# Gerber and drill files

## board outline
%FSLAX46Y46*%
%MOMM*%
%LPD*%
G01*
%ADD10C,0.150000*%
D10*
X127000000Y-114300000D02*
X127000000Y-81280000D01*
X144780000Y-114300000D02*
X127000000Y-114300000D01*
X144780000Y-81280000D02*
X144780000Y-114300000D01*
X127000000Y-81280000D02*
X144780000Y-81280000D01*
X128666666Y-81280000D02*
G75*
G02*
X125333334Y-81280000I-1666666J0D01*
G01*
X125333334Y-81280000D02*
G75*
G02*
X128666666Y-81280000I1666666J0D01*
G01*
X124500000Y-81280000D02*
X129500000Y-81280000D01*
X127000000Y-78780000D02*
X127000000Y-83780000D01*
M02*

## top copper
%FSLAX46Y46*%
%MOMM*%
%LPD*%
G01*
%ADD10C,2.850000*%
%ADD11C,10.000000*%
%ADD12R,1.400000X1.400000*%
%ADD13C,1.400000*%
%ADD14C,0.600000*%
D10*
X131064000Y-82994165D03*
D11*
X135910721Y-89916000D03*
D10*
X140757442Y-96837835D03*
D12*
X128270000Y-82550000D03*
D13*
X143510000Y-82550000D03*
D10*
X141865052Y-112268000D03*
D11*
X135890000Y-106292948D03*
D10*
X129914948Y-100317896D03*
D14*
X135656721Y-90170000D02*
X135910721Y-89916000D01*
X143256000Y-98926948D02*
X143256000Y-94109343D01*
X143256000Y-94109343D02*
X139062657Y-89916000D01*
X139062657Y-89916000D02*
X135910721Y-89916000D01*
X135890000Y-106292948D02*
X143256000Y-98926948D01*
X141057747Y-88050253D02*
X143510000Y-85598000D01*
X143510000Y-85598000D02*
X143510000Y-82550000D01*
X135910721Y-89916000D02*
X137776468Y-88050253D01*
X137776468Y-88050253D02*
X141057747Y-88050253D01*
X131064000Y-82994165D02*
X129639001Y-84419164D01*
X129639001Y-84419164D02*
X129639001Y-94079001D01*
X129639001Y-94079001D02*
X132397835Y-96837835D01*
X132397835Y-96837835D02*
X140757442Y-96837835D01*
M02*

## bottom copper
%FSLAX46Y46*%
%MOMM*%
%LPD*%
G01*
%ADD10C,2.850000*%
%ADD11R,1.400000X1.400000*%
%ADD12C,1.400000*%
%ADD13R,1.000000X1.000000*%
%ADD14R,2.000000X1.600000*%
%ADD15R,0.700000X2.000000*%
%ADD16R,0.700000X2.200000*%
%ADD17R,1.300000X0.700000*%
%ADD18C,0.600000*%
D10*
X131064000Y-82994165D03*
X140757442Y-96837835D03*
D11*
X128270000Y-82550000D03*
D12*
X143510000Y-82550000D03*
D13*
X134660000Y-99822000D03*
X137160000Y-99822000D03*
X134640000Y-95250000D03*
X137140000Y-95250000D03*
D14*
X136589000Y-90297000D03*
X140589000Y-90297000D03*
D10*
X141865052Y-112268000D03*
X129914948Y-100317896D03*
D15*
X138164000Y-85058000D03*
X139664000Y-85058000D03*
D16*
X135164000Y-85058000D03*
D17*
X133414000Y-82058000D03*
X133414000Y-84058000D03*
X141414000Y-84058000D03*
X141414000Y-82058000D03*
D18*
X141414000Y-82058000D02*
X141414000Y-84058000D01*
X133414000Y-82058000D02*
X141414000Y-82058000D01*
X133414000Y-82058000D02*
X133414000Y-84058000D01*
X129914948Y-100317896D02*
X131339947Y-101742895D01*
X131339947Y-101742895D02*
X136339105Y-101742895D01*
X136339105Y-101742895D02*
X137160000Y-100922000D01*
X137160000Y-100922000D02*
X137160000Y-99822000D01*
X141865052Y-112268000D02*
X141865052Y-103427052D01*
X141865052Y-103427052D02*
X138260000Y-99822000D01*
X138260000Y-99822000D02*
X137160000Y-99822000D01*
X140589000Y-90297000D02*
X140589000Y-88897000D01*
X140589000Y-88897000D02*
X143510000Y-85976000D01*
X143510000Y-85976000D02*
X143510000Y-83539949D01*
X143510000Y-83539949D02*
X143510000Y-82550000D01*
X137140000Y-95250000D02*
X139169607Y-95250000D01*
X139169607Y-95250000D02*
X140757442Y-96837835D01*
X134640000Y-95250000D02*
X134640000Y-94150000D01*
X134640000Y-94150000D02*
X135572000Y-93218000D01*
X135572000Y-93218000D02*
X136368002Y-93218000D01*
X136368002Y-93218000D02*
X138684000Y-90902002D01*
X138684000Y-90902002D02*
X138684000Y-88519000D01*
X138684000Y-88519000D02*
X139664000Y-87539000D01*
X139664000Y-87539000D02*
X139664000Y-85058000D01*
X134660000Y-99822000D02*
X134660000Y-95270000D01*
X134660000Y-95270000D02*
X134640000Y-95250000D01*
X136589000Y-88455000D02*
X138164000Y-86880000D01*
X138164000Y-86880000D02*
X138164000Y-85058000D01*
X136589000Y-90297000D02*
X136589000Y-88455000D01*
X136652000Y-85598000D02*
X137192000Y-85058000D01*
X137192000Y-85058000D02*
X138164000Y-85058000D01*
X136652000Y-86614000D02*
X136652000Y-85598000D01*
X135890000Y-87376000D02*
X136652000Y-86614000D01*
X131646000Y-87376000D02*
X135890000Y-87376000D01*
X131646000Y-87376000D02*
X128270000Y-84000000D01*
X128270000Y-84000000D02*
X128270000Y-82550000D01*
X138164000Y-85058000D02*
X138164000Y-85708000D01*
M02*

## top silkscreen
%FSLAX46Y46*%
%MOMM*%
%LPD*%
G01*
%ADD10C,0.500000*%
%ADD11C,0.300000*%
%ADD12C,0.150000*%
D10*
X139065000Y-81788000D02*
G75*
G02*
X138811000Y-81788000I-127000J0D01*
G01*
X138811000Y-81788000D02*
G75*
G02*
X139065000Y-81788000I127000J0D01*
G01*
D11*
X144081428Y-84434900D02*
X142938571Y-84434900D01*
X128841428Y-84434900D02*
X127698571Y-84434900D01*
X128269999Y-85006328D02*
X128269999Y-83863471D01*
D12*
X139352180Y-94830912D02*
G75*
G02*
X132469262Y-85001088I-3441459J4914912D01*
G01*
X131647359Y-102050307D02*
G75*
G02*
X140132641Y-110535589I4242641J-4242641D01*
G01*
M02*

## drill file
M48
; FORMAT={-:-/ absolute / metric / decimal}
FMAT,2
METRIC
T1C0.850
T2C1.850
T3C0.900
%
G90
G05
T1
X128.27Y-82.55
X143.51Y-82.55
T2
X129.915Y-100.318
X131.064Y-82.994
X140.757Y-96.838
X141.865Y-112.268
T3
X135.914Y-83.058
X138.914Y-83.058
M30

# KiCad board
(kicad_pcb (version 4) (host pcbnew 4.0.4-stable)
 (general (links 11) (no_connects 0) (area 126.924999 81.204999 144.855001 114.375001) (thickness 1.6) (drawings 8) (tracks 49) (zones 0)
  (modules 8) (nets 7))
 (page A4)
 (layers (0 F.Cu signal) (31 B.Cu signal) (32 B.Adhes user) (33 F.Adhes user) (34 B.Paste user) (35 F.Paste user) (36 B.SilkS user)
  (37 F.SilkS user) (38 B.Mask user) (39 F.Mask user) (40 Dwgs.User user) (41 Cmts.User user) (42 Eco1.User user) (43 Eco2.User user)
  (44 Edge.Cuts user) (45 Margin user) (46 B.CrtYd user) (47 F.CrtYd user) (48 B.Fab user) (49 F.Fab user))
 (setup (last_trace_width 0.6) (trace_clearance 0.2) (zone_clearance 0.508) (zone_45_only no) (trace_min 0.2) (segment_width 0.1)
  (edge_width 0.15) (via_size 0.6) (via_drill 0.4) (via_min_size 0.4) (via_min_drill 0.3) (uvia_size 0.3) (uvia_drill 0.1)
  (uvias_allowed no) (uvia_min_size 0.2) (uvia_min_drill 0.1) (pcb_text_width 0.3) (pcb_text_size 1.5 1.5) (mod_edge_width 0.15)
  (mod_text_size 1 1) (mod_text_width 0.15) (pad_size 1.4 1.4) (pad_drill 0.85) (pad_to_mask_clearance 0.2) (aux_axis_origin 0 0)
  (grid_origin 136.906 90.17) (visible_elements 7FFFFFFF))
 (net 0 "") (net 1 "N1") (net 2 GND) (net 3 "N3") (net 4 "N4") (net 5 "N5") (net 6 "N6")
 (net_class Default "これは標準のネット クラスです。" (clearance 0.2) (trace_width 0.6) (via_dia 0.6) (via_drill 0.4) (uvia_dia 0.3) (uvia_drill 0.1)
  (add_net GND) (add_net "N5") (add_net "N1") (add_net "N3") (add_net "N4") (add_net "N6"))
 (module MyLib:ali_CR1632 (layer F.Cu) (at 135.910721 89.916 305)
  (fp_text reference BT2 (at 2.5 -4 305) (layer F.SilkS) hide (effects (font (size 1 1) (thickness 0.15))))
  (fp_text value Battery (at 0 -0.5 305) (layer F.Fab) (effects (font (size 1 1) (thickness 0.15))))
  (fp_arc (start 0 0) (end 6 0) (angle 180) (layer F.SilkS) (width 0.15))
  (pad 1 thru_hole circle (at -8.45 0 305) (size 2.85 2.85) (drill 1.85) (layers *.Cu *.Mask) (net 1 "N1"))
  (pad 2 smd circle (at 0 0 305) (size 10 10) (layers F.Cu F.Paste F.Mask) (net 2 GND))
  (pad 1 thru_hole circle (at 8.45 0 305) (size 2.85 2.85) (drill 1.85) (layers *.Cu *.Mask) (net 1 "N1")))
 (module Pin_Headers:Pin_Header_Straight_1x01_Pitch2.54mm (layer F.Cu) (at 128.27 82.55)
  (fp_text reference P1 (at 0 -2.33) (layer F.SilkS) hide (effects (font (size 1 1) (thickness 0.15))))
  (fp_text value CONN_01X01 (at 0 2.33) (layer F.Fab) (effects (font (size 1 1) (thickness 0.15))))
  (pad 1 thru_hole rect (at 0 0) (size 1.4 1.4) (drill 0.85) (layers *.Cu *.Mask) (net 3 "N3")))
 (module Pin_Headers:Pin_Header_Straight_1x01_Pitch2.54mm (layer F.Cu) (at 143.51 82.55)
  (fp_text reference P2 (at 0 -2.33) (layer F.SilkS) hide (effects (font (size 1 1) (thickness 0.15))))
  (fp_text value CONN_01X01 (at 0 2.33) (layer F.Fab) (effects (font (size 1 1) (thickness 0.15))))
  (pad 1 thru_hole circle (at 0 0) (size 1.4 1.4) (drill 0.85) (layers *.Cu *.Mask) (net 2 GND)))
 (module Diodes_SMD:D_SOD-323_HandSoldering (layer B.Cu) (at 135.91 99.822)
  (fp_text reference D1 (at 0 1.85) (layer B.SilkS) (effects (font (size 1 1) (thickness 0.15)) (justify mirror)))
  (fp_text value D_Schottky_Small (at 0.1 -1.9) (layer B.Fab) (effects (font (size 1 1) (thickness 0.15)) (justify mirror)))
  (pad 1 smd rect (at -1.25 0) (size 1 1) (layers B.Cu B.Paste B.Mask) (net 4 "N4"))
  (pad 2 smd rect (at 1.25 0) (size 1 1) (layers B.Cu B.Paste B.Mask) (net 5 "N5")))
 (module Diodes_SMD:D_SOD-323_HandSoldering (layer B.Cu) (at 135.89 95.25)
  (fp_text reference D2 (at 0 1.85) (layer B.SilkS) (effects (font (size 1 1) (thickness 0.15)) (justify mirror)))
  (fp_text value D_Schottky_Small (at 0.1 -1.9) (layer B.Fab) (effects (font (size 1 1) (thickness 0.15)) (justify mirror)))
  (pad 1 smd rect (at -1.25 0) (size 1 1) (layers B.Cu B.Paste B.Mask) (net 4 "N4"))
  (pad 2 smd rect (at 1.25 0) (size 1 1) (layers B.Cu B.Paste B.Mask) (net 1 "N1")))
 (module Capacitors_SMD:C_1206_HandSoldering (layer B.Cu) (at 138.589 90.297)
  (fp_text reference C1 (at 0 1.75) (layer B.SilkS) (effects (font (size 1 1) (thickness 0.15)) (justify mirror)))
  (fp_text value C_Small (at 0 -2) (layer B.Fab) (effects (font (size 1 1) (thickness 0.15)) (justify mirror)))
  (pad 1 smd rect (at -2 0) (size 2 1.6) (layers B.Cu B.Paste B.Mask) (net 3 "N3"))
  (pad 2 smd rect (at 2 0) (size 2 1.6) (layers B.Cu B.Paste B.Mask) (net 2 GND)))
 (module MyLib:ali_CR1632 (layer F.Cu) (at 135.89 106.292948 135)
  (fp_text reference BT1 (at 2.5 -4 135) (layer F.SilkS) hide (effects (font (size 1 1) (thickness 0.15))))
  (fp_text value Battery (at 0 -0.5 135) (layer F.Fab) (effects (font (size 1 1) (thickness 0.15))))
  (fp_arc (start 0 0) (end 6 0) (angle 180) (layer F.SilkS) (width 0.15))
  (pad 1 thru_hole circle (at -8.45 0 135) (size 2.85 2.85) (drill 1.85) (layers *.Cu *.Mask) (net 5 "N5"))
  (pad 2 smd circle (at 0 0 135) (size 10 10) (layers F.Cu F.Paste F.Mask) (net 2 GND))
  (pad 1 thru_hole circle (at 8.45 0 135) (size 2.85 2.85) (drill 1.85) (layers *.Cu *.Mask) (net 5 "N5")))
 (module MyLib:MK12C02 (layer B.Cu) (at 137.414 83.058)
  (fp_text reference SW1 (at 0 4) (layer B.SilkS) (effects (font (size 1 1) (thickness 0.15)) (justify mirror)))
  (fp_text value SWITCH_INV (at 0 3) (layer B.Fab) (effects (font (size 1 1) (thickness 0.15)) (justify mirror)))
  (pad "" np_thru_hole circle (at 1.5 0) (size 0.9 0.9) (drill 0.9) (layers *.Cu *.Mask))
  (pad "" np_thru_hole circle (at -1.5 0) (size 0.9 0.9) (drill 0.9) (layers *.Cu *.Mask))
  (pad 2 smd rect (at 0.75 2) (size 0.7 2) (layers B.Cu B.Paste B.Mask) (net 3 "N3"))
  (pad 3 smd rect (at 2.25 2) (size 0.7 2) (layers B.Cu B.Paste B.Mask) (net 4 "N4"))
  (pad 1 smd rect (at -2.25 2) (size 0.7 2.2) (layers B.Cu B.Paste B.Mask) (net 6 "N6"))
  (pad 4 smd rect (at -4 -1 90) (size 0.7 1.3) (layers B.Cu B.Paste B.Mask))
  (pad 4 smd rect (at -4 1 90) (size 0.7 1.3) (layers B.Cu B.Paste B.Mask))
  (pad 4 smd rect (at 4 1 90) (size 0.7 1.3) (layers B.Cu B.Paste B.Mask))
  (pad 4 smd rect (at 4 -1 90) (size 0.7 1.3) (layers B.Cu B.Paste B.Mask)))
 (gr_circle (center 138.938 81.788) (end 138.938 81.915) (layer F.SilkS) (width 0.5))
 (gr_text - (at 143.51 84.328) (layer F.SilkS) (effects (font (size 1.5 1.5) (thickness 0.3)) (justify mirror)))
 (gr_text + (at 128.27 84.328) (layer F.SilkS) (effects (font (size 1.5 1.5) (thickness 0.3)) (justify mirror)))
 (gr_line (start 127 114.3) (end 127 81.28) (angle 90) (layer Edge.Cuts) (width 0.15))
 (gr_line (start 144.78 114.3) (end 127 114.3) (angle 90) (layer Edge.Cuts) (width 0.15))
 (gr_line (start 144.78 81.28) (end 144.78 114.3) (angle 90) (layer Edge.Cuts) (width 0.15))
 (gr_line (start 127 81.28) (end 144.78 81.28) (angle 90) (layer Edge.Cuts) (width 0.15))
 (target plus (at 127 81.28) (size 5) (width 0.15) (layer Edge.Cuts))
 (segment (start 141.414 82.058) (end 141.414 84.058) (width 0.6) (layer B.Cu) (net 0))
 (segment (start 133.414 82.058) (end 141.414 82.058) (width 0.6) (layer B.Cu) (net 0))
 (segment (start 133.414 82.058) (end 133.414 84.058) (width 0.6) (layer B.Cu) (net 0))
 (segment (start 129.914948 100.317896) (end 131.339947 101.742895) (width 0.6) (layer B.Cu) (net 5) (status 10))
 (segment (start 131.339947 101.742895) (end 136.339105 101.742895) (width 0.6) (layer B.Cu) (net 5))
 (segment (start 136.339105 101.742895) (end 137.16 100.922) (width 0.6) (layer B.Cu) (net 5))
 (segment (start 137.16 100.922) (end 137.16 99.822) (width 0.6) (layer B.Cu) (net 5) (status 20))
 (segment (start 141.865052 112.268) (end 141.865052 103.427052) (width 0.6) (layer B.Cu) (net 5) (status 10))
 (segment (start 141.865052 103.427052) (end 138.26 99.822) (width 0.6) (layer B.Cu) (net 5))
 (segment (start 138.26 99.822) (end 137.16 99.822) (width 0.6) (layer B.Cu) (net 5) (status 20))
 (segment (start 140.589 90.297) (end 140.589 88.897) (width 0.6) (layer B.Cu) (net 2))
 (segment (start 140.589 88.897) (end 143.51 85.976) (width 0.6) (layer B.Cu) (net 2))
 (segment (start 143.51 85.976) (end 143.51 83.539949) (width 0.6) (layer B.Cu) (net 2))
 (segment (start 143.51 83.539949) (end 143.51 82.55) (width 0.6) (layer B.Cu) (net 2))
 (segment (start 135.656721 90.17) (end 135.910721 89.916) (width 0.6) (layer F.Cu) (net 2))
 (segment (start 143.256 98.926948) (end 143.256 94.109343) (width 0.6) (layer F.Cu) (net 2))
 (segment (start 143.256 94.109343) (end 139.062657 89.916) (width 0.6) (layer F.Cu) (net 2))
 (segment (start 139.062657 89.916) (end 135.910721 89.916) (width 0.6) (layer F.Cu) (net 2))
 (segment (start 135.89 106.292948) (end 143.256 98.926948) (width 0.6) (layer F.Cu) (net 2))
 (segment (start 141.057747 88.050253) (end 143.51 85.598) (width 0.6) (layer F.Cu) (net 2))
 (segment (start 143.51 85.598) (end 143.51 82.55) (width 0.6) (layer F.Cu) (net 2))
 (segment (start 135.910721 89.916) (end 137.776468 88.050253) (width 0.6) (layer F.Cu) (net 2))
 (segment (start 137.776468 88.050253) (end 141.057747 88.050253) (width 0.6) (layer F.Cu) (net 2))
 (segment (start 131.064 82.994165) (end 129.639001 84.419164) (width 0.6) (layer F.Cu) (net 1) (status 10))
 (segment (start 129.639001 84.419164) (end 129.639001 94.079001) (width 0.6) (layer F.Cu) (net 1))
 (segment (start 129.639001 94.079001) (end 132.397835 96.837835) (width 0.6) (layer F.Cu) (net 1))
 (segment (start 132.397835 96.837835) (end 140.757442 96.837835) (width 0.6) (layer F.Cu) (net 1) (status 20))
 (segment (start 137.14 95.25) (end 139.169607 95.25) (width 0.6) (layer B.Cu) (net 1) (status 10))
 (segment (start 139.169607 95.25) (end 140.757442 96.837835) (width 0.6) (layer B.Cu) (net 1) (status 20))
 (segment (start 134.64 95.25) (end 134.64 94.15) (width 0.6) (layer B.Cu) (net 4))
 (segment (start 134.64 94.15) (end 135.572 93.218) (width 0.6) (layer B.Cu) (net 4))
 (segment (start 135.572 93.218) (end 136.368002 93.218) (width 0.6) (layer B.Cu) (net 4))
 (segment (start 136.368002 93.218) (end 138.684 90.902002) (width 0.6) (layer B.Cu) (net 4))
 (segment (start 138.684 90.902002) (end 138.684 88.519) (width 0.6) (layer B.Cu) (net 4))
 (segment (start 138.684 88.519) (end 139.664 87.539) (width 0.6) (layer B.Cu) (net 4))
 (segment (start 139.664 87.539) (end 139.664 85.058) (width 0.6) (layer B.Cu) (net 4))
 (segment (start 134.66 99.822) (end 134.66 95.27) (width 0.6) (layer B.Cu) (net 4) (status 30))
 (segment (start 134.66 95.27) (end 134.64 95.25) (width 0.6) (layer B.Cu) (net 4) (status 30))
 (segment (start 136.589 88.455) (end 138.164 86.88) (width 0.6) (layer B.Cu) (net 3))
 (segment (start 138.164 86.88) (end 138.164 85.058) (width 0.6) (layer B.Cu) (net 3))
 (segment (start 136.589 90.297) (end 136.589 88.455) (width 0.6) (layer B.Cu) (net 3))
 (segment (start 136.652 85.598) (end 137.192 85.058) (width 0.6) (layer B.Cu) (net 3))
 (segment (start 137.192 85.058) (end 138.164 85.058) (width 0.6) (layer B.Cu) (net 3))
 (segment (start 136.652 86.614) (end 136.652 85.598) (width 0.6) (layer B.Cu) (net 3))
 (segment (start 135.89 87.376) (end 136.652 86.614) (width 0.6) (layer B.Cu) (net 3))
 (segment (start 131.646 87.376) (end 135.89 87.376) (width 0.6) (layer B.Cu) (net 3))
 (segment (start 131.646 87.376) (end 128.27 84) (width 0.6) (layer B.Cu) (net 3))
 (segment (start 128.27 84) (end 128.27 82.55) (width 0.6) (layer B.Cu) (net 3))
 (segment (start 138.164 85.058) (end 138.164 85.708) (width 0.6) (layer B.Cu) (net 3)))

